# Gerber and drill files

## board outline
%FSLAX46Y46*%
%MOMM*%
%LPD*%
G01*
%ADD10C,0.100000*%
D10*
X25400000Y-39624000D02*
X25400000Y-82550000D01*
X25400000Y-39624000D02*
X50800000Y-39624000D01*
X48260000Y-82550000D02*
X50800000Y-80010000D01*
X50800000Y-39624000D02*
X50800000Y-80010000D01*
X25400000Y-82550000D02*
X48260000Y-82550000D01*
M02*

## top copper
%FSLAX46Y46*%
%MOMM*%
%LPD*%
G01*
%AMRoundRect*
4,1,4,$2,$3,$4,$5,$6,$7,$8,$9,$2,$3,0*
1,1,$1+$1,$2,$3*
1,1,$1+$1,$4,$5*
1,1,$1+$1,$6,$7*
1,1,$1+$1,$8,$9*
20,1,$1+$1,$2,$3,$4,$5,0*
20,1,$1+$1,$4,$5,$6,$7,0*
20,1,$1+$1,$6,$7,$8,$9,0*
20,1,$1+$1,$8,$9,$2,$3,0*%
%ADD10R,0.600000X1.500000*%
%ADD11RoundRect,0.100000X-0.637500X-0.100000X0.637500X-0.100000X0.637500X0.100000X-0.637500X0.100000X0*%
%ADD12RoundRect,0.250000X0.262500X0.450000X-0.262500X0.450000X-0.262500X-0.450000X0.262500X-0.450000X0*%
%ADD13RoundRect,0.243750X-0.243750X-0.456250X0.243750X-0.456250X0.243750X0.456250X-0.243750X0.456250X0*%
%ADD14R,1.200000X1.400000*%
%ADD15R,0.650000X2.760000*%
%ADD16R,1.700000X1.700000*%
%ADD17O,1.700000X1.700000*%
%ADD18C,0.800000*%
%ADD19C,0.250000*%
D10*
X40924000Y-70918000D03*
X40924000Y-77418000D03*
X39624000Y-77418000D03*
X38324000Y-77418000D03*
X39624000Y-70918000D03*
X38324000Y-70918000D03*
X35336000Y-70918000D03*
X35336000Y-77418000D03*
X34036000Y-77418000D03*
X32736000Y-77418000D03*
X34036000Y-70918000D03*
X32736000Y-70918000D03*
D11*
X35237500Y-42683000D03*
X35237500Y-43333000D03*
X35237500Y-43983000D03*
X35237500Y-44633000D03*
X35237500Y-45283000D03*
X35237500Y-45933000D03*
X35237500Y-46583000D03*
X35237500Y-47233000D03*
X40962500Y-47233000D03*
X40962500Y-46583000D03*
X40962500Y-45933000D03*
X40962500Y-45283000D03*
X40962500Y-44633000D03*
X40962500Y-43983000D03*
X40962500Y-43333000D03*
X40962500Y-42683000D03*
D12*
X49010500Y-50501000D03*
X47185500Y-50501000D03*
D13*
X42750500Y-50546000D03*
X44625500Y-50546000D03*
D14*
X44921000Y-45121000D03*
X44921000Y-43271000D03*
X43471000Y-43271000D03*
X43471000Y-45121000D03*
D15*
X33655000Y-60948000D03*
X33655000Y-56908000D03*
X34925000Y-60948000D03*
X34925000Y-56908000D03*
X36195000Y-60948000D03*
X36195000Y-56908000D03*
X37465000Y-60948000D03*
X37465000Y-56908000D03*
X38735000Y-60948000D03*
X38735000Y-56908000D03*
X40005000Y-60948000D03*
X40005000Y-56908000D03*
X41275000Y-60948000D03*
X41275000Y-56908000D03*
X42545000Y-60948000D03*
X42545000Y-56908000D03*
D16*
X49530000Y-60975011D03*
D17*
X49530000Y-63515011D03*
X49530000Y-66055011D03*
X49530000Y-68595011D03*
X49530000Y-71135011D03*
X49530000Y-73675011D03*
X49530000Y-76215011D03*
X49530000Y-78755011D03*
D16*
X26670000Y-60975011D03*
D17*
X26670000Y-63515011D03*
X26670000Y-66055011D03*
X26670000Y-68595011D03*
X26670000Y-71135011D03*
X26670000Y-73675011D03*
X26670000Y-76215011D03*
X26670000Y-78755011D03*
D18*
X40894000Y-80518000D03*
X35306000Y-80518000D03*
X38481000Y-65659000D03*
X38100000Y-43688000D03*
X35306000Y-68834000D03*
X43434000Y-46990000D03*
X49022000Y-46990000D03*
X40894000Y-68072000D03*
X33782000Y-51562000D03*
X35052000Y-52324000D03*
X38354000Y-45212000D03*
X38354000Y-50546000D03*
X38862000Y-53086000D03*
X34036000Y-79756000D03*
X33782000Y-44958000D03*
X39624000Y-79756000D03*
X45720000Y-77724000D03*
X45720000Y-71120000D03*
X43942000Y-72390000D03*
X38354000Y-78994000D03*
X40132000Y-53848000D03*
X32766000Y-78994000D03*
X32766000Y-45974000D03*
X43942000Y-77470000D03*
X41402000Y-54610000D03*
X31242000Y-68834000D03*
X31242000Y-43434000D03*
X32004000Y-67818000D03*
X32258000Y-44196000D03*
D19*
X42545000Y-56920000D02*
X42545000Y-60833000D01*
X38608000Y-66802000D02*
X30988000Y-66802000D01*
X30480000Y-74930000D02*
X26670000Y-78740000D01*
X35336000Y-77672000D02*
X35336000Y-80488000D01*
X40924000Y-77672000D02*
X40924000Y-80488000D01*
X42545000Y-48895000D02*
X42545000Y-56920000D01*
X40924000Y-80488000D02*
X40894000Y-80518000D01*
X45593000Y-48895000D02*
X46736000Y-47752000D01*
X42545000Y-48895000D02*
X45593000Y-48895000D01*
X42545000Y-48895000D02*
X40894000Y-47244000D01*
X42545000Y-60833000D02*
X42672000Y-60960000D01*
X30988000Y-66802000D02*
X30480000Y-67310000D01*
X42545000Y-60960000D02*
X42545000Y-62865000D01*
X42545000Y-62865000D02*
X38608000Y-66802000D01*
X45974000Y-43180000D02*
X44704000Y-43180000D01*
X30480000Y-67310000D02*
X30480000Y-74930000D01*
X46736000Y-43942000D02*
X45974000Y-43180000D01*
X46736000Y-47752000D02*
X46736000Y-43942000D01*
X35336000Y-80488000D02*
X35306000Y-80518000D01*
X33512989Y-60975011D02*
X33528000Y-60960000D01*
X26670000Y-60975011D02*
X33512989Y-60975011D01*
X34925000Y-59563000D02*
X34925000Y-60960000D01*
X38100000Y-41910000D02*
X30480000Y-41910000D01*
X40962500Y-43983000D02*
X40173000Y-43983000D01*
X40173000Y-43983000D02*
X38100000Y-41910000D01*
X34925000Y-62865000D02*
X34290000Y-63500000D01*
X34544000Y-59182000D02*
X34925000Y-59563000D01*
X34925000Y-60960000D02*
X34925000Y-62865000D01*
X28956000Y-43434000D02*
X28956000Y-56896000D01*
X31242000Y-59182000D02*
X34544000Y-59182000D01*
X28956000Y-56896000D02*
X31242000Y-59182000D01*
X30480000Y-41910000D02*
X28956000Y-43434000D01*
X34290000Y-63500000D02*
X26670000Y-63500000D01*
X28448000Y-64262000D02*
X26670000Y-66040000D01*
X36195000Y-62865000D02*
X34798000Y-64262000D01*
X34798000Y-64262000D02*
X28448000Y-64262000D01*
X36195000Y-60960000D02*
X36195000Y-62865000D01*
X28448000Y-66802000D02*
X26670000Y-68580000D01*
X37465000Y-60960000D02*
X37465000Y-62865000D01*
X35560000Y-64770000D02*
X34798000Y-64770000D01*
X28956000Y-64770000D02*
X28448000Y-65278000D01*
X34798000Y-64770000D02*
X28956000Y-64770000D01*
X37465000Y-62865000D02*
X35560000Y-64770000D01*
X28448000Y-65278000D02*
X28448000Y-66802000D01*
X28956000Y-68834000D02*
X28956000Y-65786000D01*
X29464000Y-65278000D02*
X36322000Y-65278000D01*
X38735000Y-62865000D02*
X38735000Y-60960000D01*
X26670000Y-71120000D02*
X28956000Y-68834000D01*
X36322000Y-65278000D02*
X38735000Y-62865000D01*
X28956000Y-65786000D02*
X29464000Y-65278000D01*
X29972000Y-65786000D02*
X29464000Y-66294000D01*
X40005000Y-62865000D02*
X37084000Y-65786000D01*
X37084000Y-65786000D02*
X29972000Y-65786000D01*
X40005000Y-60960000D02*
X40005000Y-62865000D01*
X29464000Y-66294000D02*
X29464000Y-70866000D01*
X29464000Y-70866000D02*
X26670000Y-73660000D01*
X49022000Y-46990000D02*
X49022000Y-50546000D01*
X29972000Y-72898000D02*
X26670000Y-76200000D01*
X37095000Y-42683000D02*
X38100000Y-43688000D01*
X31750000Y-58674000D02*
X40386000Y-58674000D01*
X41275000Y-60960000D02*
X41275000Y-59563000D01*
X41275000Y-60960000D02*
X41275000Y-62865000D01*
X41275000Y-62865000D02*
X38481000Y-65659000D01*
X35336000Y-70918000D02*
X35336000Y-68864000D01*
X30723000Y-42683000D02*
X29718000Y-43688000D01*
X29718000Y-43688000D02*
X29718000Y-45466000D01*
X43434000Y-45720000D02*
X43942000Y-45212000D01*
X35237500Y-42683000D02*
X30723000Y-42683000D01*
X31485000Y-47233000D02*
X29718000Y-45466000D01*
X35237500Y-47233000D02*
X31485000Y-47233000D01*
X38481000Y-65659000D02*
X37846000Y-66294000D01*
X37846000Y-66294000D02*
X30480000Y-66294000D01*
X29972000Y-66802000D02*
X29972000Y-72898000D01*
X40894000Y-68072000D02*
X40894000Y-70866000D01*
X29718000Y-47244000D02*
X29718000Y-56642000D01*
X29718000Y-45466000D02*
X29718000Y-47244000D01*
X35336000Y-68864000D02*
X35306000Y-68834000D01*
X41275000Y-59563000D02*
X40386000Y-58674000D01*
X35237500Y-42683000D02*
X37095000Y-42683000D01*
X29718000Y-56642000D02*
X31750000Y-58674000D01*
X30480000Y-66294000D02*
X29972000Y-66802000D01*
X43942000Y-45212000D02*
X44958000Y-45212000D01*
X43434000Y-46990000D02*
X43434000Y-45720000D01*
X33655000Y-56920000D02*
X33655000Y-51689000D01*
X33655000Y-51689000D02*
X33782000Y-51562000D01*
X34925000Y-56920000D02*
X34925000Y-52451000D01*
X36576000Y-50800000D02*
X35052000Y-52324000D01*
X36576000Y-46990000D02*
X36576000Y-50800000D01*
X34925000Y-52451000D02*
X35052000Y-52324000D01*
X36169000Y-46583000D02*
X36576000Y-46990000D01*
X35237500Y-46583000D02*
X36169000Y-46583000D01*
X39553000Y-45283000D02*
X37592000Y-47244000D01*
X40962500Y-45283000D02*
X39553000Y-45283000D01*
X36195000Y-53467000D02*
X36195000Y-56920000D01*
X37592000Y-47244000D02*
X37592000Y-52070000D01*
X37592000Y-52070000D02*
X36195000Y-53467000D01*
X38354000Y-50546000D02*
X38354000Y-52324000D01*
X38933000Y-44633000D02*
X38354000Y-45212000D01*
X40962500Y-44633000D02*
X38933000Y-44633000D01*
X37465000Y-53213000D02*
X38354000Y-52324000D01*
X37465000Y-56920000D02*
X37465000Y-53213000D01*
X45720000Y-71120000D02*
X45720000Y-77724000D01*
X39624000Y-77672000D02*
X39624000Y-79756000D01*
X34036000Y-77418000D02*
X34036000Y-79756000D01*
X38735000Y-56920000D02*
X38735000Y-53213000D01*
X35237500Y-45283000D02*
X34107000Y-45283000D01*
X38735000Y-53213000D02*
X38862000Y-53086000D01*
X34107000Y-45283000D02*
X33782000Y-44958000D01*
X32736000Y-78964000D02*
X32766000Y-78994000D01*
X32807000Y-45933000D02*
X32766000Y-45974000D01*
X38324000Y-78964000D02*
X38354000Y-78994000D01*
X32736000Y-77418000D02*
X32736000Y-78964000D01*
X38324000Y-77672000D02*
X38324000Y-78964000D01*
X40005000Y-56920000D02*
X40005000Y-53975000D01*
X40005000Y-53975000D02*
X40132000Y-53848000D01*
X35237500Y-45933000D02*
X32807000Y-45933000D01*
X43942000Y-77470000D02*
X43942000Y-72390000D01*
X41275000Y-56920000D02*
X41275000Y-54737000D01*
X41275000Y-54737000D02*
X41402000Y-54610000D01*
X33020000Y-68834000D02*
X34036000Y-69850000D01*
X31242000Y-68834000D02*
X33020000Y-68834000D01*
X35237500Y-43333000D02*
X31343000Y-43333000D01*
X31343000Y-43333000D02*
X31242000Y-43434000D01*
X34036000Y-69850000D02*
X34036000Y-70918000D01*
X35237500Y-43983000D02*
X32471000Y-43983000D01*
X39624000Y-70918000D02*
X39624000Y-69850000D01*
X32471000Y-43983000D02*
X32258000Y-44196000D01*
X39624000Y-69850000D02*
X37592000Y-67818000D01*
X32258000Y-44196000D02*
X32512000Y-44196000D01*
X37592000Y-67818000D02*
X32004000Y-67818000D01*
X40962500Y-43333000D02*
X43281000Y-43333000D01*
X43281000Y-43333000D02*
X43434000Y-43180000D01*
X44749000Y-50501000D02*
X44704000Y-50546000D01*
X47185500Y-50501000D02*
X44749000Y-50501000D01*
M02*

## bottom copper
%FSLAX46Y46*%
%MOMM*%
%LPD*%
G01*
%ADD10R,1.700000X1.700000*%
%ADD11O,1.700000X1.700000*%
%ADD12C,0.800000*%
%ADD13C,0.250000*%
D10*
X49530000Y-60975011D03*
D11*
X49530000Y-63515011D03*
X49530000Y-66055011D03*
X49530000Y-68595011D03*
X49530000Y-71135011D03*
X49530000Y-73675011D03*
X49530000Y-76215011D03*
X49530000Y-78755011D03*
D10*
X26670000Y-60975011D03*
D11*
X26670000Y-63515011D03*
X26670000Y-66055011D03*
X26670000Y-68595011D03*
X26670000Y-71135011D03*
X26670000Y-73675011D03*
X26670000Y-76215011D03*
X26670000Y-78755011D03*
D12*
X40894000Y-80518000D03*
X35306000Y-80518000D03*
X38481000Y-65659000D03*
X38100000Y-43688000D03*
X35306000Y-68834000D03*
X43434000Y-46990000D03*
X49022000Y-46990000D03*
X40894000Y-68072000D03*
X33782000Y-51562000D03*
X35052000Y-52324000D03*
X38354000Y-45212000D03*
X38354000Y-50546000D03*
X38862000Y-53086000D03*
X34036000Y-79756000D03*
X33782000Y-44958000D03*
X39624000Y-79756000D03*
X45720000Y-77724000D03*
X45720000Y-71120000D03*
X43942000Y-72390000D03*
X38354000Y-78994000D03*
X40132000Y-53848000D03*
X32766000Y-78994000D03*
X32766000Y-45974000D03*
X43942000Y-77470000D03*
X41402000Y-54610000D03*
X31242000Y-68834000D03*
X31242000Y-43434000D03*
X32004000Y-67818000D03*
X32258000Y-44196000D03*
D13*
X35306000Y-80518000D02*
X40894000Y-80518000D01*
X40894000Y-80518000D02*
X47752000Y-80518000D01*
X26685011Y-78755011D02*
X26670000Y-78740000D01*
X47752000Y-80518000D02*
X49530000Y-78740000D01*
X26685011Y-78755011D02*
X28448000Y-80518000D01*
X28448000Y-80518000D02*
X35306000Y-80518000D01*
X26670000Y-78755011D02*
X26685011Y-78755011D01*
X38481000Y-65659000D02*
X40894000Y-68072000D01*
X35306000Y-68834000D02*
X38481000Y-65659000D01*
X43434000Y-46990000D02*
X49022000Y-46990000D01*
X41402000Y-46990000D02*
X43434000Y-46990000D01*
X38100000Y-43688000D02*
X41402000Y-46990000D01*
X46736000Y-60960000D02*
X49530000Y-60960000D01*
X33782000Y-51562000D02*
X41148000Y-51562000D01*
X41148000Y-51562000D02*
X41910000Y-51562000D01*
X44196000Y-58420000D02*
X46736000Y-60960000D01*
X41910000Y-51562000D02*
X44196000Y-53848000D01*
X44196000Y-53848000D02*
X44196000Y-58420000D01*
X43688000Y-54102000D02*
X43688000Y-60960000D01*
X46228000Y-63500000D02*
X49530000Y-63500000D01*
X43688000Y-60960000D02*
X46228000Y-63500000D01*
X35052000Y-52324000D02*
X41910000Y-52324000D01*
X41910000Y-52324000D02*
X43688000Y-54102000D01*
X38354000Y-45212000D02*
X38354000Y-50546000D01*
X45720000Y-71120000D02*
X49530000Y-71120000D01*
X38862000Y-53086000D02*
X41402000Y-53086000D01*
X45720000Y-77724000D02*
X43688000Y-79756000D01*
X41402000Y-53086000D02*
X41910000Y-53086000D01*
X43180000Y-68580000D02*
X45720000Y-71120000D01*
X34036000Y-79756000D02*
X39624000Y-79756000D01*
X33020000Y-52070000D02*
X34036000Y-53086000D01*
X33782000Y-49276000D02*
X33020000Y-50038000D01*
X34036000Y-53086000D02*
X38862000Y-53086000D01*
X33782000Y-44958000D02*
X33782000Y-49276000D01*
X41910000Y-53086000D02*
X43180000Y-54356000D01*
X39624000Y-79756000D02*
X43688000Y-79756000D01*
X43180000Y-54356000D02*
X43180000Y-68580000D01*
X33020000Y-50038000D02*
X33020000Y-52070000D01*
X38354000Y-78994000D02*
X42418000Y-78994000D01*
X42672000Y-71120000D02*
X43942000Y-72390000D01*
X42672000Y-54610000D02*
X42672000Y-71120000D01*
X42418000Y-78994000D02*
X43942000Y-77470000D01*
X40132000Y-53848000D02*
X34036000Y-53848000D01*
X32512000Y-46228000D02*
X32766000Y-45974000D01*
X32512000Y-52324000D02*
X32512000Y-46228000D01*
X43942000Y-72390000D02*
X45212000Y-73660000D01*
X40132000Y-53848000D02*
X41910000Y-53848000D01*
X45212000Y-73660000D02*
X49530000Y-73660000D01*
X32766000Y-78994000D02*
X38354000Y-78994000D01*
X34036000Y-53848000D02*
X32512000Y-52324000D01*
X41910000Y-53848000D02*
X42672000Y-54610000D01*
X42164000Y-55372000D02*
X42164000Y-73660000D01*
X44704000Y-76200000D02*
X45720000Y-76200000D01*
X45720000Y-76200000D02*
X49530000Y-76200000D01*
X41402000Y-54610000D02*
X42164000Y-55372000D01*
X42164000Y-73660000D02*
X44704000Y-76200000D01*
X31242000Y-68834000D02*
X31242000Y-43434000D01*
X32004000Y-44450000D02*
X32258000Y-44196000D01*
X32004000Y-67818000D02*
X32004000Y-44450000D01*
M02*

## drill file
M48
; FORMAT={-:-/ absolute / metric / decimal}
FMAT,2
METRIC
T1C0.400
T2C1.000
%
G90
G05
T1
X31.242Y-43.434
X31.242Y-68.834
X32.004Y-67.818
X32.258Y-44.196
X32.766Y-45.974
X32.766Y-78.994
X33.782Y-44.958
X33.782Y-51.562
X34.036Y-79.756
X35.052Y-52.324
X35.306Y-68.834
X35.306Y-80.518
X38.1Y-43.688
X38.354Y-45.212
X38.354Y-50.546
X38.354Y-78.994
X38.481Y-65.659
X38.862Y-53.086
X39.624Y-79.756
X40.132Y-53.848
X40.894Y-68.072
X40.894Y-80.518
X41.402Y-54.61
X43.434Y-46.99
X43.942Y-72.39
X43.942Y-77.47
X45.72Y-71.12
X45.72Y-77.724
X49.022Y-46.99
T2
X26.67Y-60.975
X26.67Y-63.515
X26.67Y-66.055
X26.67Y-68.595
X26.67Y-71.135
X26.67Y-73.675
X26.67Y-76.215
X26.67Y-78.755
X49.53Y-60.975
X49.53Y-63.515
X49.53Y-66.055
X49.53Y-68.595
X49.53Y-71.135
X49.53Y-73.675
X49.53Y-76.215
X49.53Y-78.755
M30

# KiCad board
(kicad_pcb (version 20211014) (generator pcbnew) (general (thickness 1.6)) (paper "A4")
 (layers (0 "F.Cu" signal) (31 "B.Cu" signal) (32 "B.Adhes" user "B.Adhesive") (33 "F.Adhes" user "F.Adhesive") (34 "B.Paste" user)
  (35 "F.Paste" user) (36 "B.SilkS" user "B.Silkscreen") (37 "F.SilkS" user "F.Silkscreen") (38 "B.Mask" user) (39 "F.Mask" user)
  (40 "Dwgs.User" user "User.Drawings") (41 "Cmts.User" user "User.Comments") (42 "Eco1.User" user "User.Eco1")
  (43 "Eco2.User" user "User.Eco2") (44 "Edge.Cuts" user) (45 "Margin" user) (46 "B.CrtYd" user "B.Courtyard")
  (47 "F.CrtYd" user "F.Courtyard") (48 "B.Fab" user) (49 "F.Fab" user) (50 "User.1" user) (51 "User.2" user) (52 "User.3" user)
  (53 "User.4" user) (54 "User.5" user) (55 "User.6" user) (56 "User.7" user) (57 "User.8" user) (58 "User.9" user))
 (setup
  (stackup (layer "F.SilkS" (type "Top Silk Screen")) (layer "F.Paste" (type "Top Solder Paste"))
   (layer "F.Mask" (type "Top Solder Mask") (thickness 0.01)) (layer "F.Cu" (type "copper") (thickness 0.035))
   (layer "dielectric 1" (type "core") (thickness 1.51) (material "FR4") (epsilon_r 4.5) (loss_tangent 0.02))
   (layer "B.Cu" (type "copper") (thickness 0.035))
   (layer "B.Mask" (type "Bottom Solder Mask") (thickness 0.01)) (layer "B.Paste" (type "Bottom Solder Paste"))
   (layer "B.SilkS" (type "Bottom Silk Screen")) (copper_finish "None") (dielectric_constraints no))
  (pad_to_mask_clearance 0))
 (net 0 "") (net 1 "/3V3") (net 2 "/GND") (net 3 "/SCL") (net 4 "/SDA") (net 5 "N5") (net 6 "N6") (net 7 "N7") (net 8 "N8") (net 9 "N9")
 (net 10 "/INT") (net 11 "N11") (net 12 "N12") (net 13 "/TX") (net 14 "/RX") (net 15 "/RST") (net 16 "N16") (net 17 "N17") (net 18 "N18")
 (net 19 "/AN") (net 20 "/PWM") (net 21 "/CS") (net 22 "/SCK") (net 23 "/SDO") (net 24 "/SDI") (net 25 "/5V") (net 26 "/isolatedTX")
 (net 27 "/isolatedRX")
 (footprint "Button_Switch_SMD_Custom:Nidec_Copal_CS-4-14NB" (layer "F.Cu") (at 39.624 74.168 -90)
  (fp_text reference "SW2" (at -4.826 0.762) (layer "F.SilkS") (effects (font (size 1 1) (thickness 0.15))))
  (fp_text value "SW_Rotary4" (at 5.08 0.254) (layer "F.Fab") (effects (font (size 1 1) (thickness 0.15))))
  (pad "1" smd rect (at -3.25 -1.3 90) (size 1.5 0.6) (layers "F.Cu" "F.Paste" "F.Mask") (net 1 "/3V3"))
  (pad "2" smd rect (at 3.25 -1.3 90) (size 1.5 0.6) (layers "F.Cu" "F.Paste" "F.Mask") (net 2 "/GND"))
  (pad "3" smd rect (at 3.25 0 90) (size 1.5 0.6) (layers "F.Cu" "F.Paste" "F.Mask") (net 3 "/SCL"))
  (pad "4" smd rect (at 3.25 1.3 90) (size 1.5 0.6) (layers "F.Cu" "F.Paste" "F.Mask") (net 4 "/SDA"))
  (pad "C" smd rect (at -3.25 0 90) (size 1.5 0.6) (layers "F.Cu" "F.Paste" "F.Mask") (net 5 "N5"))
  (pad "NC" smd rect (at -3.25 1.3 90) (size 1.5 0.6) (layers "F.Cu" "F.Paste" "F.Mask") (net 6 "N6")))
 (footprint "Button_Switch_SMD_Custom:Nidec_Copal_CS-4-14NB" (layer "F.Cu") (at 34.036 74.168 -90)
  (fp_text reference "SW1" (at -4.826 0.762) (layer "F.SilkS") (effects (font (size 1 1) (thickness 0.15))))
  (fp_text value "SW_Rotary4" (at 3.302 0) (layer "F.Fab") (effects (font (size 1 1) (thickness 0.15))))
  (pad "1" smd rect (at -3.25 -1.3 90) (size 1.5 0.6) (layers "F.Cu" "F.Paste" "F.Mask") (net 1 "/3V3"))
  (pad "2" smd rect (at 3.25 -1.3 90) (size 1.5 0.6) (layers "F.Cu" "F.Paste" "F.Mask") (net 2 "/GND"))
  (pad "3" smd rect (at 3.25 0 90) (size 1.5 0.6) (layers "F.Cu" "F.Paste" "F.Mask") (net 3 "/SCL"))
  (pad "4" smd rect (at 3.25 1.3 90) (size 1.5 0.6) (layers "F.Cu" "F.Paste" "F.Mask") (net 4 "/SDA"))
  (pad "C" smd rect (at -3.25 0 90) (size 1.5 0.6) (layers "F.Cu" "F.Paste" "F.Mask") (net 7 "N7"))
  (pad "NC" smd rect (at -3.25 1.3 90) (size 1.5 0.6) (layers "F.Cu" "F.Paste" "F.Mask") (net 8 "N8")))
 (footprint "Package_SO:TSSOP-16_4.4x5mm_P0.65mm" (layer "F.Cu") (at 38.1 44.958)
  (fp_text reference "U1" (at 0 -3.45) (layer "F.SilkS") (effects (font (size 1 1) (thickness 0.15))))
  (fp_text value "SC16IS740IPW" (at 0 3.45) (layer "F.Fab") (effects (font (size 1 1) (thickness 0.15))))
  (pad "1" smd roundrect (at -2.8625 -2.275) (size 1.475 0.4) (layers "F.Cu" "F.Paste" "F.Mask") (roundrect_rratio 0.25) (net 1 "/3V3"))
  (pad "2" smd roundrect (at -2.8625 -1.625) (size 1.475 0.4) (layers "F.Cu" "F.Paste" "F.Mask") (roundrect_rratio 0.25) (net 7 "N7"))
  (pad "3" smd roundrect (at -2.8625 -0.975) (size 1.475 0.4) (layers "F.Cu" "F.Paste" "F.Mask") (roundrect_rratio 0.25) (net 5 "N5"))
  (pad "4" smd roundrect (at -2.8625 -0.325) (size 1.475 0.4) (layers "F.Cu" "F.Paste" "F.Mask") (roundrect_rratio 0.25) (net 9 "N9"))
  (pad "5" smd roundrect (at -2.8625 0.325) (size 1.475 0.4) (layers "F.Cu" "F.Paste" "F.Mask") (roundrect_rratio 0.25) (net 3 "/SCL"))
  (pad "6" smd roundrect (at -2.8625 0.975) (size 1.475 0.4) (layers "F.Cu" "F.Paste" "F.Mask") (roundrect_rratio 0.25) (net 4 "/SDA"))
  (pad "7" smd roundrect (at -2.8625 1.625) (size 1.475 0.4) (layers "F.Cu" "F.Paste" "F.Mask") (roundrect_rratio 0.25) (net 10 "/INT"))
  (pad "8" smd roundrect (at -2.8625 2.275) (size 1.475 0.4) (layers "F.Cu" "F.Paste" "F.Mask") (roundrect_rratio 0.25) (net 1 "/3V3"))
  (pad "9" smd roundrect (at 2.8625 2.275) (size 1.475 0.4) (layers "F.Cu" "F.Paste" "F.Mask") (roundrect_rratio 0.25) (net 2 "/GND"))
  (pad "10" smd roundrect (at 2.8625 1.625) (size 1.475 0.4) (layers "F.Cu" "F.Paste" "F.Mask") (roundrect_rratio 0.25) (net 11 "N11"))
  (pad "11" smd roundrect (at 2.8625 0.975) (size 1.475 0.4) (layers "F.Cu" "F.Paste" "F.Mask") (roundrect_rratio 0.25) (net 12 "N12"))
  (pad "12" smd roundrect (at 2.8625 0.325) (size 1.475 0.4) (layers "F.Cu" "F.Paste" "F.Mask") (roundrect_rratio 0.25) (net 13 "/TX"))
  (pad "13" smd roundrect (at 2.8625 -0.325) (size 1.475 0.4) (layers "F.Cu" "F.Paste" "F.Mask") (roundrect_rratio 0.25) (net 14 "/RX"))
  (pad "14" smd roundrect (at 2.8625 -0.975) (size 1.475 0.4) (layers "F.Cu" "F.Paste" "F.Mask") (roundrect_rratio 0.25) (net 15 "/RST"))
  (pad "15" smd roundrect (at 2.8625 -1.625) (size 1.475 0.4) (layers "F.Cu" "F.Paste" "F.Mask") (roundrect_rratio 0.25) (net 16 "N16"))
  (pad "16" smd roundrect (at 2.8625 -2.275) (size 1.475 0.4) (layers "F.Cu" "F.Paste" "F.Mask") (roundrect_rratio 0.25) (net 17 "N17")))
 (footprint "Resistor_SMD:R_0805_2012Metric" (layer "F.Cu") (at 48.098 50.501 180)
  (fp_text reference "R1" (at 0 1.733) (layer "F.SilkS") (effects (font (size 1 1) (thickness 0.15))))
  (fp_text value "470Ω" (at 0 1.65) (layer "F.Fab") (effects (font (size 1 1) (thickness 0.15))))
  (pad "1" smd roundrect (at -0.9125 0 180) (size 1.025 1.4) (layers "F.Cu" "F.Paste" "F.Mask") (roundrect_rratio 0.243902) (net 1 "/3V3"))
  (pad "2" smd roundrect (at 0.9125 0 180) (size 1.025 1.4) (layers "F.Cu" "F.Paste" "F.Mask") (roundrect_rratio 0.243902) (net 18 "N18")))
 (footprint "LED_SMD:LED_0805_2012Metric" (layer "F.Cu") (at 43.688 50.546)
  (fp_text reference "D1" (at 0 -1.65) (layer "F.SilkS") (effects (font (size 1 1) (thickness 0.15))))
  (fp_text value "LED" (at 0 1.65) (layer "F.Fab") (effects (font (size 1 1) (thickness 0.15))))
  (pad "1" smd roundrect (at -0.9375 0) (size 0.975 1.4) (layers "F.Cu" "F.Paste" "F.Mask") (roundrect_rratio 0.25) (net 2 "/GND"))
  (pad "2" smd roundrect (at 0.9375 0) (size 0.975 1.4) (layers "F.Cu" "F.Paste" "F.Mask") (roundrect_rratio 0.25) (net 18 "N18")))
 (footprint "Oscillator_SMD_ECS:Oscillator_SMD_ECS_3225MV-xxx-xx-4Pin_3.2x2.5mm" (layer "F.Cu") (at 44.196 44.196 180)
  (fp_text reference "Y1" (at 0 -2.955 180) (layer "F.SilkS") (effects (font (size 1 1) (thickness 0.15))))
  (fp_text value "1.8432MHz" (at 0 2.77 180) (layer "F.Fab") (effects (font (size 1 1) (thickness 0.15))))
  (pad "1" smd rect (at -0.725 -0.925 180) (size 1.2 1.4) (layers "F.Cu" "F.Paste" "F.Mask") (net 1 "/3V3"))
  (pad "2" smd rect (at -0.725 0.925 180) (size 1.2 1.4) (layers "F.Cu" "F.Paste" "F.Mask") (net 2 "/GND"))
  (pad "3" smd rect (at 0.725 0.925 180) (size 1.2 1.4) (layers "F.Cu" "F.Paste" "F.Mask") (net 16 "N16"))
  (pad "4" smd rect (at 0.725 -0.925 180) (size 1.2 1.4) (layers "F.Cu" "F.Paste" "F.Mask") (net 1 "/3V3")))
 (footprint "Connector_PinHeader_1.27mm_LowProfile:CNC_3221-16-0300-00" (layer "F.Cu") (at 38.1 58.928)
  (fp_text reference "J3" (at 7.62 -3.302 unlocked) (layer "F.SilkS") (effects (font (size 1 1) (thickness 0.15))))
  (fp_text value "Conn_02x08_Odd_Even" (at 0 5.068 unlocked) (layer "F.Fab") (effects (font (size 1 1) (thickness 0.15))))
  (pad "1" smd rect (at -4.445 2.02) (size 0.65 2.76) (layers "F.Cu" "F.Paste" "F.Mask") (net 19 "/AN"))
  (pad "2" smd rect (at -4.445 -2.02) (size 0.65 2.76) (layers "F.Cu" "F.Paste" "F.Mask") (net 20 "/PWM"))
  (pad "3" smd rect (at -3.175 2.02) (size 0.65 2.76) (layers "F.Cu" "F.Paste" "F.Mask") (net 15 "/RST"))
  (pad "4" smd rect (at -3.175 -2.02) (size 0.65 2.76) (layers "F.Cu" "F.Paste" "F.Mask") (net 10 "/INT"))
  (pad "5" smd rect (at -1.905 2.02) (size 0.65 2.76) (layers "F.Cu" "F.Paste" "F.Mask") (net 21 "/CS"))
  (pad "6" smd rect (at -1.905 -2.02) (size 0.65 2.76) (layers "F.Cu" "F.Paste" "F.Mask") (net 13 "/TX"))
  (pad "7" smd rect (at -0.635 2.02) (size 0.65 2.76) (layers "F.Cu" "F.Paste" "F.Mask") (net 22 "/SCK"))
  (pad "8" smd rect (at -0.635 -2.02) (size 0.65 2.76) (layers "F.Cu" "F.Paste" "F.Mask") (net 14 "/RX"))
  (pad "9" smd rect (at 0.635 2.02) (size 0.65 2.76) (layers "F.Cu" "F.Paste" "F.Mask") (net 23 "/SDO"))
  (pad "10" smd rect (at 0.635 -2.02) (size 0.65 2.76) (layers "F.Cu" "F.Paste" "F.Mask") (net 3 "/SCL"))
  (pad "11" smd rect (at 1.905 2.02) (size 0.65 2.76) (layers "F.Cu" "F.Paste" "F.Mask") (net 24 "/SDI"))
  (pad "12" smd rect (at 1.905 -2.02) (size 0.65 2.76) (layers "F.Cu" "F.Paste" "F.Mask") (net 4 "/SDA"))
  (pad "13" smd rect (at 3.175 2.02) (size 0.65 2.76) (layers "F.Cu" "F.Paste" "F.Mask") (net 1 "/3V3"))
  (pad "14" smd rect (at 3.175 -2.02) (size 0.65 2.76) (layers "F.Cu" "F.Paste" "F.Mask") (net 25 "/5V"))
  (pad "15" smd rect (at 4.445 2.02) (size 0.65 2.76) (layers "F.Cu" "F.Paste" "F.Mask") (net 2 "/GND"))
  (pad "16" smd rect (at 4.445 -2.02) (size 0.65 2.76) (layers "F.Cu" "F.Paste" "F.Mask") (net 2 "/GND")))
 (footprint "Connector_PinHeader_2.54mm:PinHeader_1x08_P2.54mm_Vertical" (layer "B.Cu") (at 49.53 60.975011 180)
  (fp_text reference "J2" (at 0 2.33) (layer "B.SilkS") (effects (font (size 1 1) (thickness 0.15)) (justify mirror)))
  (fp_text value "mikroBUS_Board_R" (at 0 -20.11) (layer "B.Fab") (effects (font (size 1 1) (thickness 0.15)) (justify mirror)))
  (pad "1" thru_hole rect (at 0 0 180) (size 1.7 1.7) (drill 1) (layers *.Cu *.Mask) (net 20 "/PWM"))
  (pad "2" thru_hole oval (at 0 -2.54 180) (size 1.7 1.7) (drill 1) (layers *.Cu *.Mask) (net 10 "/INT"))
  (pad "3" thru_hole oval (at 0 -5.08 180) (size 1.7 1.7) (drill 1) (layers *.Cu *.Mask) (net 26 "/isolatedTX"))
  (pad "4" thru_hole oval (at 0 -7.62 180) (size 1.7 1.7) (drill 1) (layers *.Cu *.Mask) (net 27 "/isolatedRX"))
  (pad "5" thru_hole oval (at 0 -10.16 180) (size 1.7 1.7) (drill 1) (layers *.Cu *.Mask) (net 3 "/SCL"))
  (pad "6" thru_hole oval (at 0 -12.7 180) (size 1.7 1.7) (drill 1) (layers *.Cu *.Mask) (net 4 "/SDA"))
  (pad "7" thru_hole oval (at 0 -15.24 180) (size 1.7 1.7) (drill 1) (layers *.Cu *.Mask) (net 25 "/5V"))
  (pad "8" thru_hole oval (at 0 -17.78 180) (size 1.7 1.7) (drill 1) (layers *.Cu *.Mask) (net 2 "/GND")))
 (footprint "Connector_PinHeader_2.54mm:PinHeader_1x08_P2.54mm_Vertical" (layer "B.Cu") (at 26.67 60.975011 180)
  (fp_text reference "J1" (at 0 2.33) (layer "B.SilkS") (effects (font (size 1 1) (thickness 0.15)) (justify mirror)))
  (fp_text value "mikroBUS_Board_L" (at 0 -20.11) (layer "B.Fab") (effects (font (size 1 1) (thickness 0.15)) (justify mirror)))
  (pad "1" thru_hole rect (at 0 0 180) (size 1.7 1.7) (drill 1) (layers *.Cu *.Mask) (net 19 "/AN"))
  (pad "2" thru_hole oval (at 0 -2.54 180) (size 1.7 1.7) (drill 1) (layers *.Cu *.Mask) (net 15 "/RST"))
  (pad "3" thru_hole oval (at 0 -5.08 180) (size 1.7 1.7) (drill 1) (layers *.Cu *.Mask) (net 21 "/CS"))
  (pad "4" thru_hole oval (at 0 -7.62 180) (size 1.7 1.7) (drill 1) (layers *.Cu *.Mask) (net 22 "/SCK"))
  (pad "5" thru_hole oval (at 0 -10.16 180) (size 1.7 1.7) (drill 1) (layers *.Cu *.Mask) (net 23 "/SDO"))
  (pad "6" thru_hole oval (at 0 -12.7 180) (size 1.7 1.7) (drill 1) (layers *.Cu *.Mask) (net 24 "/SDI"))
  (pad "7" thru_hole oval (at 0 -15.24 180) (size 1.7 1.7) (drill 1) (layers *.Cu *.Mask) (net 1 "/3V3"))
  (pad "8" thru_hole oval (at 0 -17.78 180) (size 1.7 1.7) (drill 1) (layers *.Cu *.Mask) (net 2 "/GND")))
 (gr_line (start 25.4 39.624) (end 25.4 82.55) (layer "Edge.Cuts") (width 0.1))
 (gr_line (start 25.4 39.624) (end 50.8 39.624) (layer "Edge.Cuts") (width 0.1))
 (gr_line (start 48.26 82.55) (end 50.8 80.01) (layer "Edge.Cuts") (width 0.1))
 (gr_line (start 50.8 39.624) (end 50.8 80.01) (layer "Edge.Cuts") (width 0.1))
 (gr_line (start 25.4 82.55) (end 48.26 82.55) (layer "Edge.Cuts") (width 0.1))
 (segment (start 42.545 56.92) (end 42.545 60.833) (width 0.25) (layer "F.Cu") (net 2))
 (segment (start 38.608 66.802) (end 30.988 66.802) (width 0.25) (layer "F.Cu") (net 2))
 (segment (start 30.48 74.93) (end 26.67 78.74) (width 0.25) (layer "F.Cu") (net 2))
 (segment (start 35.336 77.672) (end 35.336 80.488) (width 0.25) (layer "F.Cu") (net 2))
 (segment (start 40.924 77.672) (end 40.924 80.488) (width 0.25) (layer "F.Cu") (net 2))
 (segment (start 42.545 48.895) (end 42.545 56.92) (width 0.25) (layer "F.Cu") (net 2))
 (segment (start 40.924 80.488) (end 40.894 80.518) (width 0.25) (layer "F.Cu") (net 2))
 (segment (start 45.593 48.895) (end 46.736 47.752) (width 0.25) (layer "F.Cu") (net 2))
 (segment (start 42.545 48.895) (end 45.593 48.895) (width 0.25) (layer "F.Cu") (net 2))
 (segment (start 42.545 48.895) (end 40.894 47.244) (width 0.25) (layer "F.Cu") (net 2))
 (segment (start 42.545 60.833) (end 42.672 60.96) (width 0.25) (layer "F.Cu") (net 2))
 (segment (start 30.988 66.802) (end 30.48 67.31) (width 0.25) (layer "F.Cu") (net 2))
 (segment (start 42.545 60.96) (end 42.545 62.865) (width 0.25) (layer "F.Cu") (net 2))
 (segment (start 42.545 62.865) (end 38.608 66.802) (width 0.25) (layer "F.Cu") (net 2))
 (segment (start 45.974 43.18) (end 44.704 43.18) (width 0.25) (layer "F.Cu") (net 2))
 (segment (start 30.48 67.31) (end 30.48 74.93) (width 0.25) (layer "F.Cu") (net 2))
 (segment (start 46.736 43.942) (end 45.974 43.18) (width 0.25) (layer "F.Cu") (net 2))
 (segment (start 46.736 47.752) (end 46.736 43.942) (width 0.25) (layer "F.Cu") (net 2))
 (segment (start 35.336 80.488) (end 35.306 80.518) (width 0.25) (layer "F.Cu") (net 2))
 (via (at 40.894 80.518) (size 0.8) (drill 0.4) (layers "F.Cu" "B.Cu") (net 2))
 (via (at 35.306 80.518) (size 0.8) (drill 0.4) (layers "F.Cu" "B.Cu") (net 2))
 (segment (start 35.306 80.518) (end 40.894 80.518) (width 0.25) (layer "B.Cu") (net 2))
 (segment (start 40.894 80.518) (end 47.752 80.518) (width 0.25) (layer "B.Cu") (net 2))
 (segment (start 26.685011 78.755011) (end 26.67 78.74) (width 0.25) (layer "B.Cu") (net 2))
 (segment (start 47.752 80.518) (end 49.53 78.74) (width 0.25) (layer "B.Cu") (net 2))
 (segment (start 26.685011 78.755011) (end 28.448 80.518) (width 0.25) (layer "B.Cu") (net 2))
 (segment (start 28.448 80.518) (end 35.306 80.518) (width 0.25) (layer "B.Cu") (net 2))
 (segment (start 26.67 78.755011) (end 26.685011 78.755011) (width 0.25) (layer "B.Cu") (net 2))
 (segment (start 33.512989 60.975011) (end 33.528 60.96) (width 0.25) (layer "F.Cu") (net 19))
 (segment (start 26.67 60.975011) (end 33.512989 60.975011) (width 0.25) (layer "F.Cu") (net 19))
 (segment (start 34.925 59.563) (end 34.925 60.96) (width 0.25) (layer "F.Cu") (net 15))
 (segment (start 38.1 41.91) (end 30.48 41.91) (width 0.25) (layer "F.Cu") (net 15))
 (segment (start 40.9625 43.983) (end 40.173 43.983) (width 0.25) (layer "F.Cu") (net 15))
 (segment (start 40.173 43.983) (end 38.1 41.91) (width 0.25) (layer "F.Cu") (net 15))
 (segment (start 34.925 62.865) (end 34.29 63.5) (width 0.25) (layer "F.Cu") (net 15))
 (segment (start 34.544 59.182) (end 34.925 59.563) (width 0.25) (layer "F.Cu") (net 15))
 (segment (start 34.925 60.96) (end 34.925 62.865) (width 0.25) (layer "F.Cu") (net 15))
 (segment (start 28.956 43.434) (end 28.956 56.896) (width 0.25) (layer "F.Cu") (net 15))
 (segment (start 31.242 59.182) (end 34.544 59.182) (width 0.25) (layer "F.Cu") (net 15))
 (segment (start 28.956 56.896) (end 31.242 59.182) (width 0.25) (layer "F.Cu") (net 15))
 (segment (start 30.48 41.91) (end 28.956 43.434) (width 0.25) (layer "F.Cu") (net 15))
 (segment (start 34.29 63.5) (end 26.67 63.5) (width 0.25) (layer "F.Cu") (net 15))
 (segment (start 28.448 64.262) (end 26.67 66.04) (width 0.25) (layer "F.Cu") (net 21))
 (segment (start 36.195 62.865) (end 34.798 64.262) (width 0.25) (layer "F.Cu") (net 21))
 (segment (start 34.798 64.262) (end 28.448 64.262) (width 0.25) (layer "F.Cu") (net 21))
 (segment (start 36.195 60.96) (end 36.195 62.865) (width 0.25) (layer "F.Cu") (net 21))
 (segment (start 28.448 66.802) (end 26.67 68.58) (width 0.25) (layer "F.Cu") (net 22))
 (segment (start 37.465 60.96) (end 37.465 62.865) (width 0.25) (layer "F.Cu") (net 22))
 (segment (start 35.56 64.77) (end 34.798 64.77) (width 0.25) (layer "F.Cu") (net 22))
 (segment (start 28.956 64.77) (end 28.448 65.278) (width 0.25) (layer "F.Cu") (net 22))
 (segment (start 34.798 64.77) (end 28.956 64.77) (width 0.25) (layer "F.Cu") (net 22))
 (segment (start 37.465 62.865) (end 35.56 64.77) (width 0.25) (layer "F.Cu") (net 22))
 (segment (start 28.448 65.278) (end 28.448 66.802) (width 0.25) (layer "F.Cu") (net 22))
 (segment (start 28.956 68.834) (end 28.956 65.786) (width 0.25) (layer "F.Cu") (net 23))
 (segment (start 29.464 65.278) (end 36.322 65.278) (width 0.25) (layer "F.Cu") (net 23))
 (segment (start 38.735 62.865) (end 38.735 60.96) (width 0.25) (layer "F.Cu") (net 23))
 (segment (start 26.67 71.12) (end 28.956 68.834) (width 0.25) (layer "F.Cu") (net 23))
 (segment (start 36.322 65.278) (end 38.735 62.865) (width 0.25) (layer "F.Cu") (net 23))
 (segment (start 28.956 65.786) (end 29.464 65.278) (width 0.25) (layer "F.Cu") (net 23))
 (segment (start 29.972 65.786) (end 29.464 66.294) (width 0.25) (layer "F.Cu") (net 24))
 (segment (start 40.005 62.865) (end 37.084 65.786) (width 0.25) (layer "F.Cu") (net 24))
 (segment (start 37.084 65.786) (end 29.972 65.786) (width 0.25) (layer "F.Cu") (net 24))
 (segment (start 40.005 60.96) (end 40.005 62.865) (width 0.25) (layer "F.Cu") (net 24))
 (segment (start 29.464 66.294) (end 29.464 70.866) (width 0.25) (layer "F.Cu") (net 24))
 (segment (start 29.464 70.866) (end 26.67 73.66) (width 0.25) (layer "F.Cu") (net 24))
 (segment (start 49.022 46.99) (end 49.022 50.546) (width 0.25) (layer "F.Cu") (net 1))
 (segment (start 29.972 72.898) (end 26.67 76.2) (width 0.25) (layer "F.Cu") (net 1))
 (segment (start 37.095 42.683) (end 38.1 43.688) (width 0.25) (layer "F.Cu") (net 1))
 (segment (start 31.75 58.674) (end 40.386 58.674) (width 0.25) (layer "F.Cu") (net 1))
 (segment (start 41.275 60.96) (end 41.275 59.563) (width 0.25) (layer "F.Cu") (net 1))
 (segment (start 41.275 60.96) (end 41.275 62.865) (width 0.25) (layer "F.Cu") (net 1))
 (segment (start 41.275 62.865) (end 38.481 65.659) (width 0.25) (layer "F.Cu") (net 1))
 (segment (start 35.336 70.918) (end 35.336 68.864) (width 0.25) (layer "F.Cu") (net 1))
 (segment (start 30.723 42.683) (end 29.718 43.688) (width 0.25) (layer "F.Cu") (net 1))
 (segment (start 29.718 43.688) (end 29.718 45.466) (width 0.25) (layer "F.Cu") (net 1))
 (segment (start 43.434 45.72) (end 43.942 45.212) (width 0.25) (layer "F.Cu") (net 1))
 (segment (start 35.2375 42.683) (end 30.723 42.683) (width 0.25) (layer "F.Cu") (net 1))
 (segment (start 31.485 47.233) (end 29.718 45.466) (width 0.25) (layer "F.Cu") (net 1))
 (segment (start 35.2375 47.233) (end 31.485 47.233) (width 0.25) (layer "F.Cu") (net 1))
 (segment (start 38.481 65.659) (end 37.846 66.294) (width 0.25) (layer "F.Cu") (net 1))
 (segment (start 37.846 66.294) (end 30.48 66.294) (width 0.25) (layer "F.Cu") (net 1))
 (segment (start 29.972 66.802) (end 29.972 72.898) (width 0.25) (layer "F.Cu") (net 1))
 (segment (start 40.894 68.072) (end 40.894 70.866) (width 0.25) (layer "F.Cu") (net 1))
 (segment (start 29.718 47.244) (end 29.718 56.642) (width 0.25) (layer "F.Cu") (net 1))
 (segment (start 29.718 45.466) (end 29.718 47.244) (width 0.25) (layer "F.Cu") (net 1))
 (segment (start 35.336 68.864) (end 35.306 68.834) (width 0.25) (layer "F.Cu") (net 1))
 (segment (start 41.275 59.563) (end 40.386 58.674) (width 0.25) (layer "F.Cu") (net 1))
 (segment (start 35.2375 42.683) (end 37.095 42.683) (width 0.25) (layer "F.Cu") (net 1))
 (segment (start 29.718 56.642) (end 31.75 58.674) (width 0.25) (layer "F.Cu") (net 1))
 (segment (start 30.48 66.294) (end 29.972 66.802) (width 0.25) (layer "F.Cu") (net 1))
 (segment (start 43.942 45.212) (end 44.958 45.212) (width 0.25) (layer "F.Cu") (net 1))
 (segment (start 43.434 46.99) (end 43.434 45.72) (width 0.25) (layer "F.Cu") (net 1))
 (via (at 38.481 65.659) (size 0.8) (drill 0.4) (layers "F.Cu" "B.Cu") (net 1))
 (via (at 38.1 43.688) (size 0.8) (drill 0.4) (layers "F.Cu" "B.Cu") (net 1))
 (via (at 35.306 68.834) (size 0.8) (drill 0.4) (layers "F.Cu" "B.Cu") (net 1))
 (via (at 43.434 46.99) (size 0.8) (drill 0.4) (layers "F.Cu" "B.Cu") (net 1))
 (via (at 49.022 46.99) (size 0.8) (drill 0.4) (layers "F.Cu" "B.Cu") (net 1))
 (via (at 40.894 68.072) (size 0.8) (drill 0.4) (layers "F.Cu" "B.Cu") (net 1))
 (segment (start 38.481 65.659) (end 40.894 68.072) (width 0.25) (layer "B.Cu") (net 1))
 (segment (start 35.306 68.834) (end 38.481 65.659) (width 0.25) (layer "B.Cu") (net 1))
 (segment (start 43.434 46.99) (end 49.022 46.99) (width 0.25) (layer "B.Cu") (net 1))
 (segment (start 41.402 46.99) (end 43.434 46.99) (width 0.25) (layer "B.Cu") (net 1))
 (segment (start 38.1 43.688) (end 41.402 46.99) (width 0.25) (layer "B.Cu") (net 1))
 (segment (start 33.655 56.92) (end 33.655 51.689) (width 0.25) (layer "F.Cu") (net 20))
 (segment (start 33.655 51.689) (end 33.782 51.562) (width 0.25) (layer "F.Cu") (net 20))
 (via (at 33.782 51.562) (size 0.8) (drill 0.4) (layers "F.Cu" "B.Cu") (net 20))
 (segment (start 46.736 60.96) (end 49.53 60.96) (width 0.25) (layer "B.Cu") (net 20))
 (segment (start 33.782 51.562) (end 41.148 51.562) (width 0.25) (layer "B.Cu") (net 20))
 (segment (start 41.148 51.562) (end 41.91 51.562) (width 0.25) (layer "B.Cu") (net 20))
 (segment (start 44.196 58.42) (end 46.736 60.96) (width 0.25) (layer "B.Cu") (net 20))
 (segment (start 41.91 51.562) (end 44.196 53.848) (width 0.25) (layer "B.Cu") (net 20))
 (segment (start 44.196 53.848) (end 44.196 58.42) (width 0.25) (layer "B.Cu") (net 20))
 (segment (start 34.925 56.92) (end 34.925 52.451) (width 0.25) (layer "F.Cu") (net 10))
 (segment (start 36.576 50.8) (end 35.052 52.324) (width 0.25) (layer "F.Cu") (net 10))
 (segment (start 36.576 46.99) (end 36.576 50.8) (width 0.25) (layer "F.Cu") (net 10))
 (segment (start 34.925 52.451) (end 35.052 52.324) (width 0.25) (layer "F.Cu") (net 10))
 (segment (start 36.169 46.583) (end 36.576 46.99) (width 0.25) (layer "F.Cu") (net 10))
 (segment (start 35.2375 46.583) (end 36.169 46.583) (width 0.25) (layer "F.Cu") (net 10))
 (via (at 35.052 52.324) (size 0.8) (drill 0.4) (layers "F.Cu" "B.Cu") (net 10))
 (segment (start 43.688 54.102) (end 43.688 60.96) (width 0.25) (layer "B.Cu") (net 10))
 (segment (start 46.228 63.5) (end 49.53 63.5) (width 0.25) (layer "B.Cu") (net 10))
 (segment (start 43.688 60.96) (end 46.228 63.5) (width 0.25) (layer "B.Cu") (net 10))
 (segment (start 35.052 52.324) (end 41.91 52.324) (width 0.25) (layer "B.Cu") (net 10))
 (segment (start 41.91 52.324) (end 43.688 54.102) (width 0.25) (layer "B.Cu") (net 10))
 (segment (start 39.553 45.283) (end 37.592 47.244) (width 0.25) (layer "F.Cu") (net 13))
 (segment (start 40.9625 45.283) (end 39.553 45.283) (width 0.25) (layer "F.Cu") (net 13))
 (segment (start 36.195 53.467) (end 36.195 56.92) (width 0.25) (layer "F.Cu") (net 13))
 (segment (start 37.592 47.244) (end 37.592 52.07) (width 0.25) (layer "F.Cu") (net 13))
 (segment (start 37.592 52.07) (end 36.195 53.467) (width 0.25) (layer "F.Cu") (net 13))
 (segment (start 38.354 50.546) (end 38.354 52.324) (width 0.25) (layer "F.Cu") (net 14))
 (segment (start 38.933 44.633) (end 38.354 45.212) (width 0.25) (layer "F.Cu") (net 14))
 (segment (start 40.9625 44.633) (end 38.933 44.633) (width 0.25) (layer "F.Cu") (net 14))
 (segment (start 37.465 53.213) (end 38.354 52.324) (width 0.25) (layer "F.Cu") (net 14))
 (segment (start 37.465 56.92) (end 37.465 53.213) (width 0.25) (layer "F.Cu") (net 14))
 (via (at 38.354 45.212) (size 0.8) (drill 0.4) (layers "F.Cu" "B.Cu") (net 14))
 (via (at 38.354 50.546) (size 0.8) (drill 0.4) (layers "F.Cu" "B.Cu") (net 14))
 (segment (start 38.354 45.212) (end 38.354 50.546) (width 0.25) (layer "B.Cu") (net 14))
 (segment (start 45.72 71.12) (end 45.72 77.724) (width 0.25) (layer "F.Cu") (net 3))
 (segment (start 39.624 77.672) (end 39.624 79.756) (width 0.25) (layer "F.Cu") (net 3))
 (segment (start 34.036 77.418) (end 34.036 79.756) (width 0.25) (layer "F.Cu") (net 3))
 (segment (start 38.735 56.92) (end 38.735 53.213) (width 0.25) (layer "F.Cu") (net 3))
 (segment (start 35.2375 45.283) (end 34.107 45.283) (width 0.25) (layer "F.Cu") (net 3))
 (segment (start 38.735 53.213) (end 38.862 53.086) (width 0.25) (layer "F.Cu") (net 3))
 (segment (start 34.107 45.283) (end 33.782 44.958) (width 0.25) (layer "F.Cu") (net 3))
 (via (at 38.862 53.086) (size 0.8) (drill 0.4) (layers "F.Cu" "B.Cu") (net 3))
 (via (at 34.036 79.756) (size 0.8) (drill 0.4) (layers "F.Cu" "B.Cu") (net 3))
 (via (at 33.782 44.958) (size 0.8) (drill 0.4) (layers "F.Cu" "B.Cu") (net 3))
 (via (at 39.624 79.756) (size 0.8) (drill 0.4) (layers "F.Cu" "B.Cu") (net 3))
 (via (at 45.72 77.724) (size 0.8) (drill 0.4) (layers "F.Cu" "B.Cu") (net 3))
 (via (at 45.72 71.12) (size 0.8) (drill 0.4) (layers "F.Cu" "B.Cu") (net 3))
 (segment (start 45.72 71.12) (end 49.53 71.12) (width 0.25) (layer "B.Cu") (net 3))
 (segment (start 38.862 53.086) (end 41.402 53.086) (width 0.25) (layer "B.Cu") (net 3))
 (segment (start 45.72 77.724) (end 43.688 79.756) (width 0.25) (layer "B.Cu") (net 3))
 (segment (start 41.402 53.086) (end 41.91 53.086) (width 0.25) (layer "B.Cu") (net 3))
 (segment (start 43.18 68.58) (end 45.72 71.12) (width 0.25) (layer "B.Cu") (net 3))
 (segment (start 34.036 79.756) (end 39.624 79.756) (width 0.25) (layer "B.Cu") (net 3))
 (segment (start 33.02 52.07) (end 34.036 53.086) (width 0.25) (layer "B.Cu") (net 3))
 (segment (start 33.782 49.276) (end 33.02 50.038) (width 0.25) (layer "B.Cu") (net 3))
 (segment (start 34.036 53.086) (end 38.862 53.086) (width 0.25) (layer "B.Cu") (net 3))
 (segment (start 33.782 44.958) (end 33.782 49.276) (width 0.25) (layer "B.Cu") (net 3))
 (segment (start 41.91 53.086) (end 43.18 54.356) (width 0.25) (layer "B.Cu") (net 3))
 (segment (start 39.624 79.756) (end 43.688 79.756) (width 0.25) (layer "B.Cu") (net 3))
 (segment (start 43.18 54.356) (end 43.18 68.58) (width 0.25) (layer "B.Cu") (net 3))
 (segment (start 33.02 50.038) (end 33.02 52.07) (width 0.25) (layer "B.Cu") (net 3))
 (segment (start 32.736 78.964) (end 32.766 78.994) (width 0.25) (layer "F.Cu") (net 4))
 (segment (start 32.807 45.933) (end 32.766 45.974) (width 0.25) (layer "F.Cu") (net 4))
 (segment (start 38.324 78.964) (end 38.354 78.994) (width 0.25) (layer "F.Cu") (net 4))
 (segment (start 32.736 77.418) (end 32.736 78.964) (width 0.25) (layer "F.Cu") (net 4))
 (segment (start 38.324 77.672) (end 38.324 78.964) (width 0.25) (layer "F.Cu") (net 4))
 (segment (start 40.005 56.92) (end 40.005 53.975) (width 0.25) (layer "F.Cu") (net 4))
 (segment (start 40.005 53.975) (end 40.132 53.848) (width 0.25) (layer "F.Cu") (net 4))
 (segment (start 35.2375 45.933) (end 32.807 45.933) (width 0.25) (layer "F.Cu") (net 4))
 (segment (start 43.942 77.47) (end 43.942 72.39) (width 0.25) (layer "F.Cu") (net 4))
 (via (at 43.942 72.39) (size 0.8) (drill 0.4) (layers "F.Cu" "B.Cu") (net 4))
 (via (at 38.354 78.994) (size 0.8) (drill 0.4) (layers "F.Cu" "B.Cu") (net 4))
 (via (at 40.132 53.848) (size 0.8) (drill 0.4) (layers "F.Cu" "B.Cu") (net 4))
 (via (at 32.766 78.994) (size 0.8) (drill 0.4) (layers "F.Cu" "B.Cu") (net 4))
 (via (at 32.766 45.974) (size 0.8) (drill 0.4) (layers "F.Cu" "B.Cu") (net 4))
 (via (at 43.942 77.47) (size 0.8) (drill 0.4) (layers "F.Cu" "B.Cu") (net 4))
 (segment (start 38.354 78.994) (end 42.418 78.994) (width 0.25) (layer "B.Cu") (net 4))
 (segment (start 42.672 71.12) (end 43.942 72.39) (width 0.25) (layer "B.Cu") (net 4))
 (segment (start 42.672 54.61) (end 42.672 71.12) (width 0.25) (layer "B.Cu") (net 4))
 (segment (start 42.418 78.994) (end 43.942 77.47) (width 0.25) (layer "B.Cu") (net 4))
 (segment (start 40.132 53.848) (end 34.036 53.848) (width 0.25) (layer "B.Cu") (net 4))
 (segment (start 32.512 46.228) (end 32.766 45.974) (width 0.25) (layer "B.Cu") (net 4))
 (segment (start 32.512 52.324) (end 32.512 46.228) (width 0.25) (layer "B.Cu") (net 4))
 (segment (start 43.942 72.39) (end 45.212 73.66) (width 0.25) (layer "B.Cu") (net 4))
 (segment (start 40.132 53.848) (end 41.91 53.848) (width 0.25) (layer "B.Cu") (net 4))
 (segment (start 45.212 73.66) (end 49.53 73.66) (width 0.25) (layer "B.Cu") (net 4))
 (segment (start 32.766 78.994) (end 38.354 78.994) (width 0.25) (layer "B.Cu") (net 4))
 (segment (start 34.036 53.848) (end 32.512 52.324) (width 0.25) (layer "B.Cu") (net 4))
 (segment (start 41.91 53.848) (end 42.672 54.61) (width 0.25) (layer "B.Cu") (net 4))
 (segment (start 41.275 56.92) (end 41.275 54.737) (width 0.25) (layer "F.Cu") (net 25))
 (segment (start 41.275 54.737) (end 41.402 54.61) (width 0.25) (layer "F.Cu") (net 25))
 (via (at 41.402 54.61) (size 0.8) (drill 0.4) (layers "F.Cu" "B.Cu") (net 25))
 (segment (start 42.164 55.372) (end 42.164 73.66) (width 0.25) (layer "B.Cu") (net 25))
 (segment (start 44.704 76.2) (end 45.72 76.2) (width 0.25) (layer "B.Cu") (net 25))
 (segment (start 45.72 76.2) (end 49.53 76.2) (width 0.25) (layer "B.Cu") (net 25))
 (segment (start 41.402 54.61) (end 42.164 55.372) (width 0.25) (layer "B.Cu") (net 25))
 (segment (start 42.164 73.66) (end 44.704 76.2) (width 0.25) (layer "B.Cu") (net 25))
 (segment (start 33.02 68.834) (end 34.036 69.85) (width 0.25) (layer "F.Cu") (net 7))
 (segment (start 31.242 68.834) (end 33.02 68.834) (width 0.25) (layer "F.Cu") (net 7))
 (segment (start 35.2375 43.333) (end 31.343 43.333) (width 0.25) (layer "F.Cu") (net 7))
 (segment (start 31.343 43.333) (end 31.242 43.434) (width 0.25) (layer "F.Cu") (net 7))
 (segment (start 34.036 69.85) (end 34.036 70.918) (width 0.25) (layer "F.Cu") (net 7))
 (via (at 31.242 68.834) (size 0.8) (drill 0.4) (layers "F.Cu" "B.Cu") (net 7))
 (via (at 31.242 43.434) (size 0.8) (drill 0.4) (layers "F.Cu" "B.Cu") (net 7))
 (segment (start 31.242 68.834) (end 31.242 43.434) (width 0.25) (layer "B.Cu") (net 7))
 (segment (start 35.2375 43.983) (end 32.471 43.983) (width 0.25) (layer "F.Cu") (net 5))
 (segment (start 39.624 70.918) (end 39.624 69.85) (width 0.25) (layer "F.Cu") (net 5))
 (segment (start 32.471 43.983) (end 32.258 44.196) (width 0.25) (layer "F.Cu") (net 5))
 (segment (start 39.624 69.85) (end 37.592 67.818) (width 0.25) (layer "F.Cu") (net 5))
 (segment (start 32.258 44.196) (end 32.512 44.196) (width 0.25) (layer "F.Cu") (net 5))
 (segment (start 37.592 67.818) (end 32.004 67.818) (width 0.25) (layer "F.Cu") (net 5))
 (via (at 32.004 67.818) (size 0.8) (drill 0.4) (layers "F.Cu" "B.Cu") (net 5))
 (via (at 32.258 44.196) (size 0.8) (drill 0.4) (layers "F.Cu" "B.Cu") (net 5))
 (segment (start 32.004 44.45) (end 32.258 44.196) (width 0.25) (layer "B.Cu") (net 5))
 (segment (start 32.004 67.818) (end 32.004 44.45) (width 0.25) (layer "B.Cu") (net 5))
 (segment (start 40.9625 43.333) (end 43.281 43.333) (width 0.25) (layer "F.Cu") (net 16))
 (segment (start 43.281 43.333) (end 43.434 43.18) (width 0.25) (layer "F.Cu") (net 16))
 (segment (start 44.749 50.501) (end 44.704 50.546) (width 0.25) (layer "F.Cu") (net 18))
 (segment (start 47.1855 50.501) (end 44.749 50.501) (width 0.25) (layer "F.Cu") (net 18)))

